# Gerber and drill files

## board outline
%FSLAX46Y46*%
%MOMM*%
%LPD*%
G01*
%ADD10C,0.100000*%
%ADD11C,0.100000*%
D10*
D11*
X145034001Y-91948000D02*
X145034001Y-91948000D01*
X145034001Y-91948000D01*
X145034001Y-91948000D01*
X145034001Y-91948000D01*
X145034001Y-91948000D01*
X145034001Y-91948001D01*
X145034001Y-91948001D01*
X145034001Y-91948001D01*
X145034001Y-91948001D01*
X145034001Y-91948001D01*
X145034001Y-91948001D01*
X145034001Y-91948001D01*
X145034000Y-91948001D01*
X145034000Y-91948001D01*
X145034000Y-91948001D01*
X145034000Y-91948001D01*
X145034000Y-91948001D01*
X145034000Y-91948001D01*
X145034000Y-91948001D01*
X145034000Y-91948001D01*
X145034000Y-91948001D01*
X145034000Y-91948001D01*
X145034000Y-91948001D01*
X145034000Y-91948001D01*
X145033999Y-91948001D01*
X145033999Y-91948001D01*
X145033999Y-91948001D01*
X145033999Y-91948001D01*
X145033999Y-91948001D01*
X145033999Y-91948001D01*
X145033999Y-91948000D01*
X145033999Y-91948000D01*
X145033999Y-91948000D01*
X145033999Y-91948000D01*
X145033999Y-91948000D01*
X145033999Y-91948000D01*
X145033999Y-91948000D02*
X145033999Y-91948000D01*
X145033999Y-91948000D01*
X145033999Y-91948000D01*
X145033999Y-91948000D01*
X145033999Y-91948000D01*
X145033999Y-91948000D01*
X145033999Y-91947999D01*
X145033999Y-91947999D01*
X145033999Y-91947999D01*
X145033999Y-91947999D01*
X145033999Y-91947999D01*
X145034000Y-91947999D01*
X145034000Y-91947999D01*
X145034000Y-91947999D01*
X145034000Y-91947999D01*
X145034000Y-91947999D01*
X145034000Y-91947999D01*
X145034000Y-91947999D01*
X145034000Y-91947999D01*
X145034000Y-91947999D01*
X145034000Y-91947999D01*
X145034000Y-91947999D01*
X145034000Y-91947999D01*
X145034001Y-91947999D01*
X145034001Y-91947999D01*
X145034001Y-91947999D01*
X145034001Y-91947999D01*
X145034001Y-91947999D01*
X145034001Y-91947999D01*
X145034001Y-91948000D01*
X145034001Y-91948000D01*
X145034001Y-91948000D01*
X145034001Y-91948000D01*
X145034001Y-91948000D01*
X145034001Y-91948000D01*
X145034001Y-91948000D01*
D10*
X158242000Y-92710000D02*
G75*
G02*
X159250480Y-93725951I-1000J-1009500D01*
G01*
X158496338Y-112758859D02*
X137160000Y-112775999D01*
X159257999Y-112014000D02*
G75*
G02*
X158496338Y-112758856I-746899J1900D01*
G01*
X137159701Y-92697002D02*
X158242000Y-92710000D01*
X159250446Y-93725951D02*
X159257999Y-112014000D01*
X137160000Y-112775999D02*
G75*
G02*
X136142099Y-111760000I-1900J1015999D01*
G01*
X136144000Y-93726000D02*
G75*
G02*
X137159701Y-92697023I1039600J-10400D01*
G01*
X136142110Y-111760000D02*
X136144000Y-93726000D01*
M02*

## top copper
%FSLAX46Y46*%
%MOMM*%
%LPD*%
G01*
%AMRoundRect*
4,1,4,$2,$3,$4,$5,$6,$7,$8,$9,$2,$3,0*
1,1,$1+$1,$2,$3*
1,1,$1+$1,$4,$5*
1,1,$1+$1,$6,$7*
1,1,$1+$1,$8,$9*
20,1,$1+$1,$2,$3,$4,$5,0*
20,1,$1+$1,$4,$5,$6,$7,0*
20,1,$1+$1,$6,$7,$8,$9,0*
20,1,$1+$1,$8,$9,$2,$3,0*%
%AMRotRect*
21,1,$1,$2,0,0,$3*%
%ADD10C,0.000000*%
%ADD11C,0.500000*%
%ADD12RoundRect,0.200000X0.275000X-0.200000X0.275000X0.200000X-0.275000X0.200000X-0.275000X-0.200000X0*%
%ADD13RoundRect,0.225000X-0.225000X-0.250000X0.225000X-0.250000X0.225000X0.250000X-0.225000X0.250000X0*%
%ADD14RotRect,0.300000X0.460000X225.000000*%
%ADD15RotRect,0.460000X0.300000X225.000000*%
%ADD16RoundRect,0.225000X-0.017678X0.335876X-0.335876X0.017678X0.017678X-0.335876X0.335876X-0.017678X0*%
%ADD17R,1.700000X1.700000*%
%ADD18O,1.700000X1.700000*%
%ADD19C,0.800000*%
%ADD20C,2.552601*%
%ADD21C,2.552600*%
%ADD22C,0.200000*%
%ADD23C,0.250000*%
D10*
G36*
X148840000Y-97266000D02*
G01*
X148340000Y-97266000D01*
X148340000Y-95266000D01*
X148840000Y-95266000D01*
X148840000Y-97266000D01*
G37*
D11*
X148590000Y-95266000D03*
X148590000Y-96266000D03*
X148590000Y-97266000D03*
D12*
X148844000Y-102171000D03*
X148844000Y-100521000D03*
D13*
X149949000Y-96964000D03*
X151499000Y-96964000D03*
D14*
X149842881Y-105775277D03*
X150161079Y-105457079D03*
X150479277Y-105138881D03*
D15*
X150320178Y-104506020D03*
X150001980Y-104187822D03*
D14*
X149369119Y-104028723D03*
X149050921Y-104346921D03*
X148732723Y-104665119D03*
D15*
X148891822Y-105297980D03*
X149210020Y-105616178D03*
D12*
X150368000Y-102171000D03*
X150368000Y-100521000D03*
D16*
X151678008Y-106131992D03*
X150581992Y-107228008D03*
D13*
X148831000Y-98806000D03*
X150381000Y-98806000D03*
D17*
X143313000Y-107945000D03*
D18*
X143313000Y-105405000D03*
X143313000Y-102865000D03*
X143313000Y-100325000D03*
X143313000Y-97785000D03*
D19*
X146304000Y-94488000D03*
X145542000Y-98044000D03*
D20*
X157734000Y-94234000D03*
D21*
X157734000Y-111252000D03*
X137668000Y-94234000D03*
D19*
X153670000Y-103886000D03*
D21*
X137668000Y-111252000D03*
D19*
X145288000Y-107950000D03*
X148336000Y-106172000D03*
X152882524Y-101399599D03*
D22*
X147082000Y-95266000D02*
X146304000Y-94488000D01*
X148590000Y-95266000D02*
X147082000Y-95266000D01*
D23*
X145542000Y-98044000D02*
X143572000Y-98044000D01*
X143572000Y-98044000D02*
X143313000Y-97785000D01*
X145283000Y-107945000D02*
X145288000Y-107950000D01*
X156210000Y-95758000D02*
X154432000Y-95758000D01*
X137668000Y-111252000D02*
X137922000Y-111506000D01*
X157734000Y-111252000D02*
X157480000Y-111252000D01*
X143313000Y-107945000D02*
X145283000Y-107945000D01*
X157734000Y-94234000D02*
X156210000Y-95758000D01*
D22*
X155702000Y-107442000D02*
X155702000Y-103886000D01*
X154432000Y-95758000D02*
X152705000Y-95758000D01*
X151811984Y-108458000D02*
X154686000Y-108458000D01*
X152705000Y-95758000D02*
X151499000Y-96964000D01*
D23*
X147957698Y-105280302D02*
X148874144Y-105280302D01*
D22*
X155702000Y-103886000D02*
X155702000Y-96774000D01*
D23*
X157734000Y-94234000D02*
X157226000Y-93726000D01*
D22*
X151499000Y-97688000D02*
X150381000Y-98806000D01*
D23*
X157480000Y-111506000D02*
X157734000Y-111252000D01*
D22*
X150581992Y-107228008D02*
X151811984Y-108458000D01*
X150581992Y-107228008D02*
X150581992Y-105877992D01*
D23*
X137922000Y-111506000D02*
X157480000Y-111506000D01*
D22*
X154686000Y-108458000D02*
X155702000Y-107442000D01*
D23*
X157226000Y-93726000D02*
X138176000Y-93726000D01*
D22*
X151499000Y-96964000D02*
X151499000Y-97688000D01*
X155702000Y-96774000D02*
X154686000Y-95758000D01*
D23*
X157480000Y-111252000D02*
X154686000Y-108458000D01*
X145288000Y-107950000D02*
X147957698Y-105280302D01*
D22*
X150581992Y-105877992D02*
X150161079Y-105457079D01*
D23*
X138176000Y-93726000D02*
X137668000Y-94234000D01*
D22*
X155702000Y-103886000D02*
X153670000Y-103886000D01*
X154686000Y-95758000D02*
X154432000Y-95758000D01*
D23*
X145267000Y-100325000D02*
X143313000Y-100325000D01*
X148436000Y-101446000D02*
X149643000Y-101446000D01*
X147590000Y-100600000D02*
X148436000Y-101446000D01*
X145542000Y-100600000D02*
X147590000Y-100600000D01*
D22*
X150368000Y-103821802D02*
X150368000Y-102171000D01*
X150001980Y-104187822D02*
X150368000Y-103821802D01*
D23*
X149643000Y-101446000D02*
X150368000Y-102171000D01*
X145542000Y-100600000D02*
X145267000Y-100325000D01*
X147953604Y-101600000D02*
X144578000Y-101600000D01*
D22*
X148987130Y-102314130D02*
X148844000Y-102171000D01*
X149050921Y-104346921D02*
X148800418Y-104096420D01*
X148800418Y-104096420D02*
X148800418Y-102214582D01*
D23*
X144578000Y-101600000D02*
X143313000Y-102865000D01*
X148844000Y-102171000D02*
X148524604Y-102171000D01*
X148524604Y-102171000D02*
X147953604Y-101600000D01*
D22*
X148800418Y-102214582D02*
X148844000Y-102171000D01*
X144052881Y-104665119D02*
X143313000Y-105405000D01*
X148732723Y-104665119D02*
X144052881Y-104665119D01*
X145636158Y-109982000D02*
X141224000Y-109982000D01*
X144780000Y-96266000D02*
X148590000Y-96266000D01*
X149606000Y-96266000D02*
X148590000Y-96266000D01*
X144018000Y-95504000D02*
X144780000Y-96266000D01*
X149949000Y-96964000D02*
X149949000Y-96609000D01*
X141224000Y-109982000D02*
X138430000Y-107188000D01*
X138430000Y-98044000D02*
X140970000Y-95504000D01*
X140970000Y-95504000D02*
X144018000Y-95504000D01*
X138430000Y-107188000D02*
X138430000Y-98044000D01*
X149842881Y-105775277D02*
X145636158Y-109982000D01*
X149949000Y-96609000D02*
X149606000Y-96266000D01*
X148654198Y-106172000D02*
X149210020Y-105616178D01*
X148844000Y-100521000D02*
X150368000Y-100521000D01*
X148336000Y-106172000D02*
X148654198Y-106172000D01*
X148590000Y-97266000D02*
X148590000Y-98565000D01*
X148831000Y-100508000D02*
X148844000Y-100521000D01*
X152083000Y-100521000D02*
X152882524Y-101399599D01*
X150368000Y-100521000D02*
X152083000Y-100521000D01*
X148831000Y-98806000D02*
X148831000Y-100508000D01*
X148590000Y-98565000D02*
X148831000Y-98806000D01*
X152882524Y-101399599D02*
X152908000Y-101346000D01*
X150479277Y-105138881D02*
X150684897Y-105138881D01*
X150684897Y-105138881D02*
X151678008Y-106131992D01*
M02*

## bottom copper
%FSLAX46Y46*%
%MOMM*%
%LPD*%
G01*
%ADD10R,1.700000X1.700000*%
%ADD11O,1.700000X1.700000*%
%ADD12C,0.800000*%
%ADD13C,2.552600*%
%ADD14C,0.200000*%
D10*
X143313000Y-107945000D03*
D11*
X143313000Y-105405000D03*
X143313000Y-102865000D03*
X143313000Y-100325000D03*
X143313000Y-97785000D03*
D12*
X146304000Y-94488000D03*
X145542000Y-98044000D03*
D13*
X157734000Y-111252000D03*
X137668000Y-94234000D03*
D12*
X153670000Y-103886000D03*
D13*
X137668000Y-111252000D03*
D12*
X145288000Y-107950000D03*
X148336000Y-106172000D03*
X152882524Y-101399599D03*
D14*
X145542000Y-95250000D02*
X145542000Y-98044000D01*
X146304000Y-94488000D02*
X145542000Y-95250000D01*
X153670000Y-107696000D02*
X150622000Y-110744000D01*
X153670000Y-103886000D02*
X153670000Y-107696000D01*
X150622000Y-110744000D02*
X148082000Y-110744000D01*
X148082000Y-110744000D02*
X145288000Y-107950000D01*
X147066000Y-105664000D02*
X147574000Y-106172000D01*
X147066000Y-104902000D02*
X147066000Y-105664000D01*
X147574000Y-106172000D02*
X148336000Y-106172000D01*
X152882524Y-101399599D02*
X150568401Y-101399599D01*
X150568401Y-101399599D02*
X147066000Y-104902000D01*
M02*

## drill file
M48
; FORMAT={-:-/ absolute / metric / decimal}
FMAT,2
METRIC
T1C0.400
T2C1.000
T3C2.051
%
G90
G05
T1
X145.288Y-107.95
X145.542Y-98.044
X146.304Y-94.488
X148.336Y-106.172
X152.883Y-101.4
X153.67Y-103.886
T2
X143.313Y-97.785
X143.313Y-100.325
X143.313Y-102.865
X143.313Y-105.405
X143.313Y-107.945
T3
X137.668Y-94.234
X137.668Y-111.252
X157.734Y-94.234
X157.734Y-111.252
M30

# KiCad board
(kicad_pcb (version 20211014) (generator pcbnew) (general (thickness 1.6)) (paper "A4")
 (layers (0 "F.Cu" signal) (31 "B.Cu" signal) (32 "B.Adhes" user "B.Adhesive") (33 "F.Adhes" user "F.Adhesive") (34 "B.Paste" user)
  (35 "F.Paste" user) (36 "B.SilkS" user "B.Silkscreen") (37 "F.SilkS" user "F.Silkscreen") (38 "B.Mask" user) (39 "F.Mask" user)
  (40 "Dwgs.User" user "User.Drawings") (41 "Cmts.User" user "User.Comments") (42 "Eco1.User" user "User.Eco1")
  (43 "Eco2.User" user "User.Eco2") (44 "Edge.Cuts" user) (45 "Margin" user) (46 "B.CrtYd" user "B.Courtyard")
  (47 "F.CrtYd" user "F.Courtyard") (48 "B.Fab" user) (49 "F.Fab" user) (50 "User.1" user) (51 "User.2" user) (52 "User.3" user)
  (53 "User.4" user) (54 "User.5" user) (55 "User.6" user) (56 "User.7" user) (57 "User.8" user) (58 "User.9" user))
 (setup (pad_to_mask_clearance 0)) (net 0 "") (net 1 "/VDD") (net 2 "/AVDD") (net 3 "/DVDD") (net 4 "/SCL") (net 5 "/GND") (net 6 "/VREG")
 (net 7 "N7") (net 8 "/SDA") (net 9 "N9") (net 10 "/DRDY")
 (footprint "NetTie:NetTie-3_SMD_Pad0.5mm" (layer "F.Cu") (at 148.59 96.266 -90)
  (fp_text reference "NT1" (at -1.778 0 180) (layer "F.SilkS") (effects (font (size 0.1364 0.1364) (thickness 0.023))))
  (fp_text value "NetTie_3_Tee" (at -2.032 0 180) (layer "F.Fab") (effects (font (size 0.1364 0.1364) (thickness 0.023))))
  (fp_poly (pts (xy -1 -0.25) (xy 1 -0.25) (xy 1 0.25) (xy -1 0.25)) (layer "F.Cu") (width 0) (fill solid))
  (pad "1" smd circle (at -1 0 270) (size 0.5 0.5) (layers "F.Cu") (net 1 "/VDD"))
  (pad "2" smd circle (at 0 0 270) (size 0.5 0.5) (layers "F.Cu") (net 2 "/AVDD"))
  (pad "3" smd circle (at 1 0 270) (size 0.5 0.5) (layers "F.Cu") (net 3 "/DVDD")))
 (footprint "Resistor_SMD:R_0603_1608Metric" (layer "F.Cu") (at 148.844 101.346 90)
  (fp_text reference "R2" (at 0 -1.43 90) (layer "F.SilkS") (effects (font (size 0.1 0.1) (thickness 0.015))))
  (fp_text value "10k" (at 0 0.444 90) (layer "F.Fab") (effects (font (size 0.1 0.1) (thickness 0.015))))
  (pad "1" smd roundrect (at -0.825 0 90) (size 0.8 0.95) (layers "F.Cu" "F.Paste" "F.Mask") (roundrect_rratio 0.25) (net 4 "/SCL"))
  (pad "2" smd roundrect (at 0.825 0 90) (size 0.8 0.95) (layers "F.Cu" "F.Paste" "F.Mask") (roundrect_rratio 0.25) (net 3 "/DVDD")))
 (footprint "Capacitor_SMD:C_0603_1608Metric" (layer "F.Cu") (at 150.724 96.964)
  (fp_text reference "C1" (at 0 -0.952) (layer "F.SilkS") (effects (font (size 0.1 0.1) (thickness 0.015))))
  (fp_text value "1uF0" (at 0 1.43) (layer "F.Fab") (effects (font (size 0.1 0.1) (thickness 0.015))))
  (pad "1" smd roundrect (at -0.775 0) (size 0.9 0.95) (layers "F.Cu" "F.Paste" "F.Mask") (roundrect_rratio 0.25) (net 2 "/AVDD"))
  (pad "2" smd roundrect (at 0.775 0) (size 0.9 0.95) (layers "F.Cu" "F.Paste" "F.Mask") (roundrect_rratio 0.25) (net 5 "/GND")))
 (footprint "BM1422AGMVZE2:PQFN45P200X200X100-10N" (layer "F.Cu") (at 149.606 104.902 135)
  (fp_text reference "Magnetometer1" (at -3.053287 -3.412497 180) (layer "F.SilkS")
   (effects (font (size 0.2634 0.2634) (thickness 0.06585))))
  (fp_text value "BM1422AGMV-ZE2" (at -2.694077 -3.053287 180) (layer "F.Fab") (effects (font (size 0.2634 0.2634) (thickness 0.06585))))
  (pad "1" smd rect locked (at -0.785 -0.45 225) (size 0.3 0.46) (layers "F.Cu" "F.Paste" "F.Mask") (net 2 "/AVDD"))
  (pad "2" smd rect locked (at -0.785 0 225) (size 0.3 0.46) (layers "F.Cu" "F.Paste" "F.Mask") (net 5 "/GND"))
  (pad "3" smd rect locked (at -0.785 0.45 225) (size 0.3 0.46) (layers "F.Cu" "F.Paste" "F.Mask") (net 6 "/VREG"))
  (pad "4" smd rect locked (at -0.225 0.785 225) (size 0.46 0.3) (layers "F.Cu" "F.Paste" "F.Mask") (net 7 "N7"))
  (pad "5" smd rect locked (at 0.225 0.785 225) (size 0.46 0.3) (layers "F.Cu" "F.Paste" "F.Mask") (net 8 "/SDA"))
  (pad "6" smd rect locked (at 0.785 0.45 225) (size 0.3 0.46) (layers "F.Cu" "F.Paste" "F.Mask") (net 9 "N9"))
  (pad "7" smd rect locked (at 0.785 0 225) (size 0.3 0.46) (layers "F.Cu" "F.Paste" "F.Mask") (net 4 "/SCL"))
  (pad "8" smd rect locked (at 0.785 -0.45 225) (size 0.3 0.46) (layers "F.Cu" "F.Paste" "F.Mask") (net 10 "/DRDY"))
  (pad "9" smd rect locked (at 0.225 -0.785 225) (size 0.46 0.3) (layers "F.Cu" "F.Paste" "F.Mask") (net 5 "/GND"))
  (pad "10" smd rect locked (at -0.225 -0.785 225) (size 0.46 0.3) (layers "F.Cu" "F.Paste" "F.Mask") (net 3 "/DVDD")))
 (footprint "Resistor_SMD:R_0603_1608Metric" (layer "F.Cu") (at 150.368 101.346 90)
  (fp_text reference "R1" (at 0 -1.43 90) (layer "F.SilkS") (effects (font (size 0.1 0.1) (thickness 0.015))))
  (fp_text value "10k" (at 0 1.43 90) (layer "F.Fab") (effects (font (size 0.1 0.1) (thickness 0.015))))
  (pad "1" smd roundrect (at -0.825 0 90) (size 0.8 0.95) (layers "F.Cu" "F.Paste" "F.Mask") (roundrect_rratio 0.25) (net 8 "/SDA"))
  (pad "2" smd roundrect (at 0.825 0 90) (size 0.8 0.95) (layers "F.Cu" "F.Paste" "F.Mask") (roundrect_rratio 0.25) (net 3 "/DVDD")))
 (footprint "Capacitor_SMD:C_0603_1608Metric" (layer "F.Cu") (at 151.13 106.68 -135)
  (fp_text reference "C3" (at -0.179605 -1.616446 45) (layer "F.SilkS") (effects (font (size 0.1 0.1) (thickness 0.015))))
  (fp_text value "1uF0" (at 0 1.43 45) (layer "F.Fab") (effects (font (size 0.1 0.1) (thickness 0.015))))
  (pad "1" smd roundrect (at -0.775 0 225) (size 0.9 0.95) (layers "F.Cu" "F.Paste" "F.Mask") (roundrect_rratio 0.25) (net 6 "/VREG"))
  (pad "2" smd roundrect (at 0.775 0 225) (size 0.9 0.95) (layers "F.Cu" "F.Paste" "F.Mask") (roundrect_rratio 0.25) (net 5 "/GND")))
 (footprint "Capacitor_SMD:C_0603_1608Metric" (layer "F.Cu") (at 149.606 98.806)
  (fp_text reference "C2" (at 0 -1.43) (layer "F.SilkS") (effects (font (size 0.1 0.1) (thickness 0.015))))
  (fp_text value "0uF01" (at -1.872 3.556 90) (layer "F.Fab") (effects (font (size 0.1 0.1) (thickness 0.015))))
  (pad "1" smd roundrect (at -0.775 0) (size 0.9 0.95) (layers "F.Cu" "F.Paste" "F.Mask") (roundrect_rratio 0.25) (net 3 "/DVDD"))
  (pad "2" smd roundrect (at 0.775 0) (size 0.9 0.95) (layers "F.Cu" "F.Paste" "F.Mask") (roundrect_rratio 0.25) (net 5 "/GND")))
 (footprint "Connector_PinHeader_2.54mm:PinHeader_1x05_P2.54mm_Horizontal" (layer "F.Cu") (at 143.313 107.945 180)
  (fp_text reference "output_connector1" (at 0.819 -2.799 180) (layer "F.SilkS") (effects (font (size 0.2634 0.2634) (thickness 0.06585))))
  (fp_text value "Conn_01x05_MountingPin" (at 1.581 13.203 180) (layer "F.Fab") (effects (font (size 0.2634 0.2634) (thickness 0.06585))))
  (pad "1" thru_hole rect (at 0 0 180) (size 1.7 1.7) (drill 1) (layers *.Cu *.Mask) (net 5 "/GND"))
  (pad "2" thru_hole oval (at 0 2.54 180) (size 1.7 1.7) (drill 1) (layers *.Cu *.Mask) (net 10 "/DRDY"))
  (pad "3" thru_hole oval (at 0 5.08 180) (size 1.7 1.7) (drill 1) (layers *.Cu *.Mask) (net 4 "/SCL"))
  (pad "4" thru_hole oval (at 0 7.62 180) (size 1.7 1.7) (drill 1) (layers *.Cu *.Mask) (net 8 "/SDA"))
  (pad "5" thru_hole oval (at 0 10.16 180) (size 1.7 1.7) (drill 1) (layers *.Cu *.Mask) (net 1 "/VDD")))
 (gr_circle (center 145.034 91.948) (end 145.034 91.948) (layer "Edge.Cuts") (width 0.1) (fill none))
 (gr_arc (start 158.242 92.71) (mid 158.957418 93.008321) (end 159.250446 93.725951) (layer "Edge.Cuts") (width 0.1))
 (gr_line (start 158.496338 112.758859) (end 137.16 112.775999) (layer "Edge.Cuts") (width 0.1))
 (gr_arc (start 159.257999 112.014) (mid 159.033315 112.546097) (end 158.496338 112.758859) (layer "Edge.Cuts") (width 0.1))
 (gr_line (start 137.159701 92.697002) (end 158.242 92.71) (layer "Edge.Cuts") (width 0.1))
 (gr_line (start 159.250446 93.725951) (end 159.257999 112.014) (layer "Edge.Cuts") (width 0.1))
 (gr_arc (start 137.16 112.775999) (mid 136.440351 112.479092) (end 136.14211 111.76) (layer "Edge.Cuts") (width 0.1))
 (gr_arc (start 136.144 93.726) (mid 136.443697 93.006044) (end 137.159701 92.697002) (layer "Edge.Cuts") (width 0.1))
 (gr_line (start 136.14211 111.76) (end 136.144 93.726) (layer "Edge.Cuts") (width 0.1))
 (segment (start 147.082 95.266) (end 146.304 94.488) (width 0.2) (layer "F.Cu") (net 1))
 (segment (start 148.59 95.266) (end 147.082 95.266) (width 0.2) (layer "F.Cu") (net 1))
 (segment (start 145.542 98.044) (end 143.572 98.044) (width 0.25) (layer "F.Cu") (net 1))
 (segment (start 143.572 98.044) (end 143.313 97.785) (width 0.25) (layer "F.Cu") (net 1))
 (via (at 146.304 94.488) (size 0.8) (drill 0.4) (layers "F.Cu" "B.Cu") (free) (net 1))
 (via (at 145.542 98.044) (size 0.8) (drill 0.4) (layers "F.Cu" "B.Cu") (free) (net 1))
 (segment (start 145.542 95.25) (end 145.542 98.044) (width 0.2) (layer "B.Cu") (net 1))
 (segment (start 146.304 94.488) (end 145.542 95.25) (width 0.2) (layer "B.Cu") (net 1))
 (segment (start 145.283 107.945) (end 145.288 107.95) (width 0.25) (layer "F.Cu") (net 5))
 (segment (start 156.21 95.758) (end 154.432 95.758) (width 0.25) (layer "F.Cu") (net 5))
 (segment (start 137.668 111.252) (end 137.922 111.506) (width 0.25) (layer "F.Cu") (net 5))
 (segment (start 157.734 111.252) (end 157.48 111.252) (width 0.25) (layer "F.Cu") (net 5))
 (segment (start 143.313 107.945) (end 145.283 107.945) (width 0.25) (layer "F.Cu") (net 5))
 (segment (start 157.734 94.234) (end 156.21 95.758) (width 0.25) (layer "F.Cu") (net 5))
 (segment (start 155.702 107.442) (end 155.702 103.886) (width 0.2) (layer "F.Cu") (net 5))
 (segment (start 154.432 95.758) (end 152.705 95.758) (width 0.2) (layer "F.Cu") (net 5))
 (segment (start 151.811984 108.458) (end 154.686 108.458) (width 0.2) (layer "F.Cu") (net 5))
 (segment (start 152.705 95.758) (end 151.499 96.964) (width 0.2) (layer "F.Cu") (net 5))
 (segment (start 147.957698 105.280302) (end 148.874144 105.280302) (width 0.25) (layer "F.Cu") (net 5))
 (segment (start 155.702 103.886) (end 155.702 96.774) (width 0.2) (layer "F.Cu") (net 5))
 (segment (start 157.734 94.234) (end 157.226 93.726) (width 0.25) (layer "F.Cu") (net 5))
 (segment (start 151.499 97.688) (end 150.381 98.806) (width 0.2) (layer "F.Cu") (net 5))
 (segment (start 157.48 111.506) (end 157.734 111.252) (width 0.25) (layer "F.Cu") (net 5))
 (segment (start 150.581992 107.228008) (end 151.811984 108.458) (width 0.2) (layer "F.Cu") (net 5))
 (segment (start 150.581992 107.228008) (end 150.581992 105.877992) (width 0.2) (layer "F.Cu") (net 5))
 (segment (start 137.922 111.506) (end 157.48 111.506) (width 0.25) (layer "F.Cu") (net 5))
 (segment (start 154.686 108.458) (end 155.702 107.442) (width 0.2) (layer "F.Cu") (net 5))
 (segment (start 157.226 93.726) (end 138.176 93.726) (width 0.25) (layer "F.Cu") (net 5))
 (segment (start 151.499 96.964) (end 151.499 97.688) (width 0.2) (layer "F.Cu") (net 5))
 (segment (start 155.702 96.774) (end 154.686 95.758) (width 0.2) (layer "F.Cu") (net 5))
 (segment (start 157.48 111.252) (end 154.686 108.458) (width 0.25) (layer "F.Cu") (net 5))
 (segment (start 145.288 107.95) (end 147.957698 105.280302) (width 0.25) (layer "F.Cu") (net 5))
 (segment (start 150.581992 105.877992) (end 150.161079 105.457079) (width 0.2) (layer "F.Cu") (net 5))
 (segment (start 138.176 93.726) (end 137.668 94.234) (width 0.25) (layer "F.Cu") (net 5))
 (segment (start 155.702 103.886) (end 153.67 103.886) (width 0.2) (layer "F.Cu") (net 5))
 (segment (start 154.686 95.758) (end 154.432 95.758) (width 0.2) (layer "F.Cu") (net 5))
 (via (at 157.734 94.234) (size 2.552601) (drill 2.051) (layers "F.Cu" "B.Cu") (remove_unused_layers) (free) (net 5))
 (via (at 157.734 111.252) (size 2.5526) (drill 2.051) (layers "F.Cu" "B.Cu") (free) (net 5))
 (via (at 137.668 94.234) (size 2.5526) (drill 2.051) (layers "F.Cu" "B.Cu") (free) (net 5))
 (via (at 153.67 103.886) (size 0.8) (drill 0.4) (layers "F.Cu" "B.Cu") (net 5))
 (via (at 137.668 111.252) (size 2.5526) (drill 2.051) (layers "F.Cu" "B.Cu") (free) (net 5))
 (via (at 145.288 107.95) (size 0.8) (drill 0.4) (layers "F.Cu" "B.Cu") (free) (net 5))
 (segment (start 153.67 107.696) (end 150.622 110.744) (width 0.2) (layer "B.Cu") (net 5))
 (segment (start 153.67 103.886) (end 153.67 107.696) (width 0.2) (layer "B.Cu") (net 5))
 (segment (start 150.622 110.744) (end 148.082 110.744) (width 0.2) (layer "B.Cu") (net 5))
 (segment (start 148.082 110.744) (end 145.288 107.95) (width 0.2) (layer "B.Cu") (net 5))
 (segment (start 145.267 100.325) (end 143.313 100.325) (width 0.25) (layer "F.Cu") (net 8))
 (segment (start 148.436 101.446) (end 149.643 101.446) (width 0.25) (layer "F.Cu") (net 8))
 (segment (start 147.59 100.6) (end 148.436 101.446) (width 0.25) (layer "F.Cu") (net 8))
 (segment (start 145.542 100.6) (end 147.59 100.6) (width 0.25) (layer "F.Cu") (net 8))
 (segment (start 150.368 103.821802) (end 150.368 102.171) (width 0.2) (layer "F.Cu") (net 8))
 (segment (start 150.00198 104.187822) (end 150.368 103.821802) (width 0.2) (layer "F.Cu") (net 8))
 (segment (start 149.643 101.446) (end 150.368 102.171) (width 0.25) (layer "F.Cu") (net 8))
 (segment (start 145.542 100.6) (end 145.267 100.325) (width 0.25) (layer "F.Cu") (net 8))
 (segment (start 147.953604 101.6) (end 144.578 101.6) (width 0.25) (layer "F.Cu") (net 4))
 (segment (start 148.98713 102.31413) (end 148.844 102.171) (width 0.2) (layer "F.Cu") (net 4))
 (segment (start 149.050921 104.346921) (end 148.800418 104.09642) (width 0.2) (layer "F.Cu") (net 4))
 (segment (start 148.800418 104.09642) (end 148.800418 102.214582) (width 0.2) (layer "F.Cu") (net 4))
 (segment (start 144.578 101.6) (end 143.313 102.865) (width 0.25) (layer "F.Cu") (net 4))
 (segment (start 148.844 102.171) (end 148.524604 102.171) (width 0.25) (layer "F.Cu") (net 4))
 (segment (start 148.524604 102.171) (end 147.953604 101.6) (width 0.25) (layer "F.Cu") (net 4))
 (segment (start 148.800418 102.214582) (end 148.844 102.171) (width 0.2) (layer "F.Cu") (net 4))
 (segment (start 144.052881 104.665119) (end 143.313 105.405) (width 0.2) (layer "F.Cu") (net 10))
 (segment (start 148.732723 104.665119) (end 144.052881 104.665119) (width 0.2) (layer "F.Cu") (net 10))
 (segment (start 145.636158 109.982) (end 141.224 109.982) (width 0.2) (layer "F.Cu") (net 2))
 (segment (start 144.78 96.266) (end 148.59 96.266) (width 0.2) (layer "F.Cu") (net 2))
 (segment (start 149.606 96.266) (end 148.59 96.266) (width 0.2) (layer "F.Cu") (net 2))
 (segment (start 144.018 95.504) (end 144.78 96.266) (width 0.2) (layer "F.Cu") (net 2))
 (segment (start 149.949 96.964) (end 149.949 96.609) (width 0.2) (layer "F.Cu") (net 2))
 (segment (start 141.224 109.982) (end 138.43 107.188) (width 0.2) (layer "F.Cu") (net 2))
 (segment (start 138.43 98.044) (end 140.97 95.504) (width 0.2) (layer "F.Cu") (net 2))
 (segment (start 140.97 95.504) (end 144.018 95.504) (width 0.2) (layer "F.Cu") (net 2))
 (segment (start 138.43 107.188) (end 138.43 98.044) (width 0.2) (layer "F.Cu") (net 2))
 (segment (start 149.842881 105.775277) (end 145.636158 109.982) (width 0.2) (layer "F.Cu") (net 2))
 (segment (start 149.949 96.609) (end 149.606 96.266) (width 0.2) (layer "F.Cu") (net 2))
 (segment (start 148.654198 106.172) (end 149.21002 105.616178) (width 0.2) (layer "F.Cu") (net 3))
 (segment (start 148.844 100.521) (end 150.368 100.521) (width 0.2) (layer "F.Cu") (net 3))
 (segment (start 148.336 106.172) (end 148.654198 106.172) (width 0.2) (layer "F.Cu") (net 3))
 (segment (start 148.59 97.266) (end 148.59 98.565) (width 0.2) (layer "F.Cu") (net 3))
 (segment (start 148.831 100.508) (end 148.844 100.521) (width 0.2) (layer "F.Cu") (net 3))
 (segment (start 152.083 100.521) (end 152.882524 101.399599) (width 0.2) (layer "F.Cu") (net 3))
 (segment (start 150.368 100.521) (end 152.083 100.521) (width 0.2) (layer "F.Cu") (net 3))
 (segment (start 148.831 98.806) (end 148.831 100.508) (width 0.2) (layer "F.Cu") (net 3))
 (segment (start 148.59 98.565) (end 148.831 98.806) (width 0.2) (layer "F.Cu") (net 3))
 (segment (start 152.882524 101.399599) (end 152.908 101.346) (width 0.2) (layer "F.Cu") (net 3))
 (via (at 148.336 106.172) (size 0.8) (drill 0.4) (layers "F.Cu" "B.Cu") (free) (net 3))
 (via (at 152.882524 101.399599) (size 0.8) (drill 0.4) (layers "F.Cu" "B.Cu") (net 3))
 (segment (start 147.066 105.664) (end 147.574 106.172) (width 0.2) (layer "B.Cu") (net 3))
 (segment (start 147.066 104.902) (end 147.066 105.664) (width 0.2) (layer "B.Cu") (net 3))
 (segment (start 147.574 106.172) (end 148.336 106.172) (width 0.2) (layer "B.Cu") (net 3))
 (segment (start 152.882524 101.399599) (end 150.568401 101.399599) (width 0.2) (layer "B.Cu") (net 3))
 (segment (start 150.568401 101.399599) (end 147.066 104.902) (width 0.2) (layer "B.Cu") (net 3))
 (segment (start 150.479277 105.138881) (end 150.684897 105.138881) (width 0.2) (layer "F.Cu") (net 6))
 (segment (start 150.684897 105.138881) (end 151.678008 106.131992) (width 0.2) (layer "F.Cu") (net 6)))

